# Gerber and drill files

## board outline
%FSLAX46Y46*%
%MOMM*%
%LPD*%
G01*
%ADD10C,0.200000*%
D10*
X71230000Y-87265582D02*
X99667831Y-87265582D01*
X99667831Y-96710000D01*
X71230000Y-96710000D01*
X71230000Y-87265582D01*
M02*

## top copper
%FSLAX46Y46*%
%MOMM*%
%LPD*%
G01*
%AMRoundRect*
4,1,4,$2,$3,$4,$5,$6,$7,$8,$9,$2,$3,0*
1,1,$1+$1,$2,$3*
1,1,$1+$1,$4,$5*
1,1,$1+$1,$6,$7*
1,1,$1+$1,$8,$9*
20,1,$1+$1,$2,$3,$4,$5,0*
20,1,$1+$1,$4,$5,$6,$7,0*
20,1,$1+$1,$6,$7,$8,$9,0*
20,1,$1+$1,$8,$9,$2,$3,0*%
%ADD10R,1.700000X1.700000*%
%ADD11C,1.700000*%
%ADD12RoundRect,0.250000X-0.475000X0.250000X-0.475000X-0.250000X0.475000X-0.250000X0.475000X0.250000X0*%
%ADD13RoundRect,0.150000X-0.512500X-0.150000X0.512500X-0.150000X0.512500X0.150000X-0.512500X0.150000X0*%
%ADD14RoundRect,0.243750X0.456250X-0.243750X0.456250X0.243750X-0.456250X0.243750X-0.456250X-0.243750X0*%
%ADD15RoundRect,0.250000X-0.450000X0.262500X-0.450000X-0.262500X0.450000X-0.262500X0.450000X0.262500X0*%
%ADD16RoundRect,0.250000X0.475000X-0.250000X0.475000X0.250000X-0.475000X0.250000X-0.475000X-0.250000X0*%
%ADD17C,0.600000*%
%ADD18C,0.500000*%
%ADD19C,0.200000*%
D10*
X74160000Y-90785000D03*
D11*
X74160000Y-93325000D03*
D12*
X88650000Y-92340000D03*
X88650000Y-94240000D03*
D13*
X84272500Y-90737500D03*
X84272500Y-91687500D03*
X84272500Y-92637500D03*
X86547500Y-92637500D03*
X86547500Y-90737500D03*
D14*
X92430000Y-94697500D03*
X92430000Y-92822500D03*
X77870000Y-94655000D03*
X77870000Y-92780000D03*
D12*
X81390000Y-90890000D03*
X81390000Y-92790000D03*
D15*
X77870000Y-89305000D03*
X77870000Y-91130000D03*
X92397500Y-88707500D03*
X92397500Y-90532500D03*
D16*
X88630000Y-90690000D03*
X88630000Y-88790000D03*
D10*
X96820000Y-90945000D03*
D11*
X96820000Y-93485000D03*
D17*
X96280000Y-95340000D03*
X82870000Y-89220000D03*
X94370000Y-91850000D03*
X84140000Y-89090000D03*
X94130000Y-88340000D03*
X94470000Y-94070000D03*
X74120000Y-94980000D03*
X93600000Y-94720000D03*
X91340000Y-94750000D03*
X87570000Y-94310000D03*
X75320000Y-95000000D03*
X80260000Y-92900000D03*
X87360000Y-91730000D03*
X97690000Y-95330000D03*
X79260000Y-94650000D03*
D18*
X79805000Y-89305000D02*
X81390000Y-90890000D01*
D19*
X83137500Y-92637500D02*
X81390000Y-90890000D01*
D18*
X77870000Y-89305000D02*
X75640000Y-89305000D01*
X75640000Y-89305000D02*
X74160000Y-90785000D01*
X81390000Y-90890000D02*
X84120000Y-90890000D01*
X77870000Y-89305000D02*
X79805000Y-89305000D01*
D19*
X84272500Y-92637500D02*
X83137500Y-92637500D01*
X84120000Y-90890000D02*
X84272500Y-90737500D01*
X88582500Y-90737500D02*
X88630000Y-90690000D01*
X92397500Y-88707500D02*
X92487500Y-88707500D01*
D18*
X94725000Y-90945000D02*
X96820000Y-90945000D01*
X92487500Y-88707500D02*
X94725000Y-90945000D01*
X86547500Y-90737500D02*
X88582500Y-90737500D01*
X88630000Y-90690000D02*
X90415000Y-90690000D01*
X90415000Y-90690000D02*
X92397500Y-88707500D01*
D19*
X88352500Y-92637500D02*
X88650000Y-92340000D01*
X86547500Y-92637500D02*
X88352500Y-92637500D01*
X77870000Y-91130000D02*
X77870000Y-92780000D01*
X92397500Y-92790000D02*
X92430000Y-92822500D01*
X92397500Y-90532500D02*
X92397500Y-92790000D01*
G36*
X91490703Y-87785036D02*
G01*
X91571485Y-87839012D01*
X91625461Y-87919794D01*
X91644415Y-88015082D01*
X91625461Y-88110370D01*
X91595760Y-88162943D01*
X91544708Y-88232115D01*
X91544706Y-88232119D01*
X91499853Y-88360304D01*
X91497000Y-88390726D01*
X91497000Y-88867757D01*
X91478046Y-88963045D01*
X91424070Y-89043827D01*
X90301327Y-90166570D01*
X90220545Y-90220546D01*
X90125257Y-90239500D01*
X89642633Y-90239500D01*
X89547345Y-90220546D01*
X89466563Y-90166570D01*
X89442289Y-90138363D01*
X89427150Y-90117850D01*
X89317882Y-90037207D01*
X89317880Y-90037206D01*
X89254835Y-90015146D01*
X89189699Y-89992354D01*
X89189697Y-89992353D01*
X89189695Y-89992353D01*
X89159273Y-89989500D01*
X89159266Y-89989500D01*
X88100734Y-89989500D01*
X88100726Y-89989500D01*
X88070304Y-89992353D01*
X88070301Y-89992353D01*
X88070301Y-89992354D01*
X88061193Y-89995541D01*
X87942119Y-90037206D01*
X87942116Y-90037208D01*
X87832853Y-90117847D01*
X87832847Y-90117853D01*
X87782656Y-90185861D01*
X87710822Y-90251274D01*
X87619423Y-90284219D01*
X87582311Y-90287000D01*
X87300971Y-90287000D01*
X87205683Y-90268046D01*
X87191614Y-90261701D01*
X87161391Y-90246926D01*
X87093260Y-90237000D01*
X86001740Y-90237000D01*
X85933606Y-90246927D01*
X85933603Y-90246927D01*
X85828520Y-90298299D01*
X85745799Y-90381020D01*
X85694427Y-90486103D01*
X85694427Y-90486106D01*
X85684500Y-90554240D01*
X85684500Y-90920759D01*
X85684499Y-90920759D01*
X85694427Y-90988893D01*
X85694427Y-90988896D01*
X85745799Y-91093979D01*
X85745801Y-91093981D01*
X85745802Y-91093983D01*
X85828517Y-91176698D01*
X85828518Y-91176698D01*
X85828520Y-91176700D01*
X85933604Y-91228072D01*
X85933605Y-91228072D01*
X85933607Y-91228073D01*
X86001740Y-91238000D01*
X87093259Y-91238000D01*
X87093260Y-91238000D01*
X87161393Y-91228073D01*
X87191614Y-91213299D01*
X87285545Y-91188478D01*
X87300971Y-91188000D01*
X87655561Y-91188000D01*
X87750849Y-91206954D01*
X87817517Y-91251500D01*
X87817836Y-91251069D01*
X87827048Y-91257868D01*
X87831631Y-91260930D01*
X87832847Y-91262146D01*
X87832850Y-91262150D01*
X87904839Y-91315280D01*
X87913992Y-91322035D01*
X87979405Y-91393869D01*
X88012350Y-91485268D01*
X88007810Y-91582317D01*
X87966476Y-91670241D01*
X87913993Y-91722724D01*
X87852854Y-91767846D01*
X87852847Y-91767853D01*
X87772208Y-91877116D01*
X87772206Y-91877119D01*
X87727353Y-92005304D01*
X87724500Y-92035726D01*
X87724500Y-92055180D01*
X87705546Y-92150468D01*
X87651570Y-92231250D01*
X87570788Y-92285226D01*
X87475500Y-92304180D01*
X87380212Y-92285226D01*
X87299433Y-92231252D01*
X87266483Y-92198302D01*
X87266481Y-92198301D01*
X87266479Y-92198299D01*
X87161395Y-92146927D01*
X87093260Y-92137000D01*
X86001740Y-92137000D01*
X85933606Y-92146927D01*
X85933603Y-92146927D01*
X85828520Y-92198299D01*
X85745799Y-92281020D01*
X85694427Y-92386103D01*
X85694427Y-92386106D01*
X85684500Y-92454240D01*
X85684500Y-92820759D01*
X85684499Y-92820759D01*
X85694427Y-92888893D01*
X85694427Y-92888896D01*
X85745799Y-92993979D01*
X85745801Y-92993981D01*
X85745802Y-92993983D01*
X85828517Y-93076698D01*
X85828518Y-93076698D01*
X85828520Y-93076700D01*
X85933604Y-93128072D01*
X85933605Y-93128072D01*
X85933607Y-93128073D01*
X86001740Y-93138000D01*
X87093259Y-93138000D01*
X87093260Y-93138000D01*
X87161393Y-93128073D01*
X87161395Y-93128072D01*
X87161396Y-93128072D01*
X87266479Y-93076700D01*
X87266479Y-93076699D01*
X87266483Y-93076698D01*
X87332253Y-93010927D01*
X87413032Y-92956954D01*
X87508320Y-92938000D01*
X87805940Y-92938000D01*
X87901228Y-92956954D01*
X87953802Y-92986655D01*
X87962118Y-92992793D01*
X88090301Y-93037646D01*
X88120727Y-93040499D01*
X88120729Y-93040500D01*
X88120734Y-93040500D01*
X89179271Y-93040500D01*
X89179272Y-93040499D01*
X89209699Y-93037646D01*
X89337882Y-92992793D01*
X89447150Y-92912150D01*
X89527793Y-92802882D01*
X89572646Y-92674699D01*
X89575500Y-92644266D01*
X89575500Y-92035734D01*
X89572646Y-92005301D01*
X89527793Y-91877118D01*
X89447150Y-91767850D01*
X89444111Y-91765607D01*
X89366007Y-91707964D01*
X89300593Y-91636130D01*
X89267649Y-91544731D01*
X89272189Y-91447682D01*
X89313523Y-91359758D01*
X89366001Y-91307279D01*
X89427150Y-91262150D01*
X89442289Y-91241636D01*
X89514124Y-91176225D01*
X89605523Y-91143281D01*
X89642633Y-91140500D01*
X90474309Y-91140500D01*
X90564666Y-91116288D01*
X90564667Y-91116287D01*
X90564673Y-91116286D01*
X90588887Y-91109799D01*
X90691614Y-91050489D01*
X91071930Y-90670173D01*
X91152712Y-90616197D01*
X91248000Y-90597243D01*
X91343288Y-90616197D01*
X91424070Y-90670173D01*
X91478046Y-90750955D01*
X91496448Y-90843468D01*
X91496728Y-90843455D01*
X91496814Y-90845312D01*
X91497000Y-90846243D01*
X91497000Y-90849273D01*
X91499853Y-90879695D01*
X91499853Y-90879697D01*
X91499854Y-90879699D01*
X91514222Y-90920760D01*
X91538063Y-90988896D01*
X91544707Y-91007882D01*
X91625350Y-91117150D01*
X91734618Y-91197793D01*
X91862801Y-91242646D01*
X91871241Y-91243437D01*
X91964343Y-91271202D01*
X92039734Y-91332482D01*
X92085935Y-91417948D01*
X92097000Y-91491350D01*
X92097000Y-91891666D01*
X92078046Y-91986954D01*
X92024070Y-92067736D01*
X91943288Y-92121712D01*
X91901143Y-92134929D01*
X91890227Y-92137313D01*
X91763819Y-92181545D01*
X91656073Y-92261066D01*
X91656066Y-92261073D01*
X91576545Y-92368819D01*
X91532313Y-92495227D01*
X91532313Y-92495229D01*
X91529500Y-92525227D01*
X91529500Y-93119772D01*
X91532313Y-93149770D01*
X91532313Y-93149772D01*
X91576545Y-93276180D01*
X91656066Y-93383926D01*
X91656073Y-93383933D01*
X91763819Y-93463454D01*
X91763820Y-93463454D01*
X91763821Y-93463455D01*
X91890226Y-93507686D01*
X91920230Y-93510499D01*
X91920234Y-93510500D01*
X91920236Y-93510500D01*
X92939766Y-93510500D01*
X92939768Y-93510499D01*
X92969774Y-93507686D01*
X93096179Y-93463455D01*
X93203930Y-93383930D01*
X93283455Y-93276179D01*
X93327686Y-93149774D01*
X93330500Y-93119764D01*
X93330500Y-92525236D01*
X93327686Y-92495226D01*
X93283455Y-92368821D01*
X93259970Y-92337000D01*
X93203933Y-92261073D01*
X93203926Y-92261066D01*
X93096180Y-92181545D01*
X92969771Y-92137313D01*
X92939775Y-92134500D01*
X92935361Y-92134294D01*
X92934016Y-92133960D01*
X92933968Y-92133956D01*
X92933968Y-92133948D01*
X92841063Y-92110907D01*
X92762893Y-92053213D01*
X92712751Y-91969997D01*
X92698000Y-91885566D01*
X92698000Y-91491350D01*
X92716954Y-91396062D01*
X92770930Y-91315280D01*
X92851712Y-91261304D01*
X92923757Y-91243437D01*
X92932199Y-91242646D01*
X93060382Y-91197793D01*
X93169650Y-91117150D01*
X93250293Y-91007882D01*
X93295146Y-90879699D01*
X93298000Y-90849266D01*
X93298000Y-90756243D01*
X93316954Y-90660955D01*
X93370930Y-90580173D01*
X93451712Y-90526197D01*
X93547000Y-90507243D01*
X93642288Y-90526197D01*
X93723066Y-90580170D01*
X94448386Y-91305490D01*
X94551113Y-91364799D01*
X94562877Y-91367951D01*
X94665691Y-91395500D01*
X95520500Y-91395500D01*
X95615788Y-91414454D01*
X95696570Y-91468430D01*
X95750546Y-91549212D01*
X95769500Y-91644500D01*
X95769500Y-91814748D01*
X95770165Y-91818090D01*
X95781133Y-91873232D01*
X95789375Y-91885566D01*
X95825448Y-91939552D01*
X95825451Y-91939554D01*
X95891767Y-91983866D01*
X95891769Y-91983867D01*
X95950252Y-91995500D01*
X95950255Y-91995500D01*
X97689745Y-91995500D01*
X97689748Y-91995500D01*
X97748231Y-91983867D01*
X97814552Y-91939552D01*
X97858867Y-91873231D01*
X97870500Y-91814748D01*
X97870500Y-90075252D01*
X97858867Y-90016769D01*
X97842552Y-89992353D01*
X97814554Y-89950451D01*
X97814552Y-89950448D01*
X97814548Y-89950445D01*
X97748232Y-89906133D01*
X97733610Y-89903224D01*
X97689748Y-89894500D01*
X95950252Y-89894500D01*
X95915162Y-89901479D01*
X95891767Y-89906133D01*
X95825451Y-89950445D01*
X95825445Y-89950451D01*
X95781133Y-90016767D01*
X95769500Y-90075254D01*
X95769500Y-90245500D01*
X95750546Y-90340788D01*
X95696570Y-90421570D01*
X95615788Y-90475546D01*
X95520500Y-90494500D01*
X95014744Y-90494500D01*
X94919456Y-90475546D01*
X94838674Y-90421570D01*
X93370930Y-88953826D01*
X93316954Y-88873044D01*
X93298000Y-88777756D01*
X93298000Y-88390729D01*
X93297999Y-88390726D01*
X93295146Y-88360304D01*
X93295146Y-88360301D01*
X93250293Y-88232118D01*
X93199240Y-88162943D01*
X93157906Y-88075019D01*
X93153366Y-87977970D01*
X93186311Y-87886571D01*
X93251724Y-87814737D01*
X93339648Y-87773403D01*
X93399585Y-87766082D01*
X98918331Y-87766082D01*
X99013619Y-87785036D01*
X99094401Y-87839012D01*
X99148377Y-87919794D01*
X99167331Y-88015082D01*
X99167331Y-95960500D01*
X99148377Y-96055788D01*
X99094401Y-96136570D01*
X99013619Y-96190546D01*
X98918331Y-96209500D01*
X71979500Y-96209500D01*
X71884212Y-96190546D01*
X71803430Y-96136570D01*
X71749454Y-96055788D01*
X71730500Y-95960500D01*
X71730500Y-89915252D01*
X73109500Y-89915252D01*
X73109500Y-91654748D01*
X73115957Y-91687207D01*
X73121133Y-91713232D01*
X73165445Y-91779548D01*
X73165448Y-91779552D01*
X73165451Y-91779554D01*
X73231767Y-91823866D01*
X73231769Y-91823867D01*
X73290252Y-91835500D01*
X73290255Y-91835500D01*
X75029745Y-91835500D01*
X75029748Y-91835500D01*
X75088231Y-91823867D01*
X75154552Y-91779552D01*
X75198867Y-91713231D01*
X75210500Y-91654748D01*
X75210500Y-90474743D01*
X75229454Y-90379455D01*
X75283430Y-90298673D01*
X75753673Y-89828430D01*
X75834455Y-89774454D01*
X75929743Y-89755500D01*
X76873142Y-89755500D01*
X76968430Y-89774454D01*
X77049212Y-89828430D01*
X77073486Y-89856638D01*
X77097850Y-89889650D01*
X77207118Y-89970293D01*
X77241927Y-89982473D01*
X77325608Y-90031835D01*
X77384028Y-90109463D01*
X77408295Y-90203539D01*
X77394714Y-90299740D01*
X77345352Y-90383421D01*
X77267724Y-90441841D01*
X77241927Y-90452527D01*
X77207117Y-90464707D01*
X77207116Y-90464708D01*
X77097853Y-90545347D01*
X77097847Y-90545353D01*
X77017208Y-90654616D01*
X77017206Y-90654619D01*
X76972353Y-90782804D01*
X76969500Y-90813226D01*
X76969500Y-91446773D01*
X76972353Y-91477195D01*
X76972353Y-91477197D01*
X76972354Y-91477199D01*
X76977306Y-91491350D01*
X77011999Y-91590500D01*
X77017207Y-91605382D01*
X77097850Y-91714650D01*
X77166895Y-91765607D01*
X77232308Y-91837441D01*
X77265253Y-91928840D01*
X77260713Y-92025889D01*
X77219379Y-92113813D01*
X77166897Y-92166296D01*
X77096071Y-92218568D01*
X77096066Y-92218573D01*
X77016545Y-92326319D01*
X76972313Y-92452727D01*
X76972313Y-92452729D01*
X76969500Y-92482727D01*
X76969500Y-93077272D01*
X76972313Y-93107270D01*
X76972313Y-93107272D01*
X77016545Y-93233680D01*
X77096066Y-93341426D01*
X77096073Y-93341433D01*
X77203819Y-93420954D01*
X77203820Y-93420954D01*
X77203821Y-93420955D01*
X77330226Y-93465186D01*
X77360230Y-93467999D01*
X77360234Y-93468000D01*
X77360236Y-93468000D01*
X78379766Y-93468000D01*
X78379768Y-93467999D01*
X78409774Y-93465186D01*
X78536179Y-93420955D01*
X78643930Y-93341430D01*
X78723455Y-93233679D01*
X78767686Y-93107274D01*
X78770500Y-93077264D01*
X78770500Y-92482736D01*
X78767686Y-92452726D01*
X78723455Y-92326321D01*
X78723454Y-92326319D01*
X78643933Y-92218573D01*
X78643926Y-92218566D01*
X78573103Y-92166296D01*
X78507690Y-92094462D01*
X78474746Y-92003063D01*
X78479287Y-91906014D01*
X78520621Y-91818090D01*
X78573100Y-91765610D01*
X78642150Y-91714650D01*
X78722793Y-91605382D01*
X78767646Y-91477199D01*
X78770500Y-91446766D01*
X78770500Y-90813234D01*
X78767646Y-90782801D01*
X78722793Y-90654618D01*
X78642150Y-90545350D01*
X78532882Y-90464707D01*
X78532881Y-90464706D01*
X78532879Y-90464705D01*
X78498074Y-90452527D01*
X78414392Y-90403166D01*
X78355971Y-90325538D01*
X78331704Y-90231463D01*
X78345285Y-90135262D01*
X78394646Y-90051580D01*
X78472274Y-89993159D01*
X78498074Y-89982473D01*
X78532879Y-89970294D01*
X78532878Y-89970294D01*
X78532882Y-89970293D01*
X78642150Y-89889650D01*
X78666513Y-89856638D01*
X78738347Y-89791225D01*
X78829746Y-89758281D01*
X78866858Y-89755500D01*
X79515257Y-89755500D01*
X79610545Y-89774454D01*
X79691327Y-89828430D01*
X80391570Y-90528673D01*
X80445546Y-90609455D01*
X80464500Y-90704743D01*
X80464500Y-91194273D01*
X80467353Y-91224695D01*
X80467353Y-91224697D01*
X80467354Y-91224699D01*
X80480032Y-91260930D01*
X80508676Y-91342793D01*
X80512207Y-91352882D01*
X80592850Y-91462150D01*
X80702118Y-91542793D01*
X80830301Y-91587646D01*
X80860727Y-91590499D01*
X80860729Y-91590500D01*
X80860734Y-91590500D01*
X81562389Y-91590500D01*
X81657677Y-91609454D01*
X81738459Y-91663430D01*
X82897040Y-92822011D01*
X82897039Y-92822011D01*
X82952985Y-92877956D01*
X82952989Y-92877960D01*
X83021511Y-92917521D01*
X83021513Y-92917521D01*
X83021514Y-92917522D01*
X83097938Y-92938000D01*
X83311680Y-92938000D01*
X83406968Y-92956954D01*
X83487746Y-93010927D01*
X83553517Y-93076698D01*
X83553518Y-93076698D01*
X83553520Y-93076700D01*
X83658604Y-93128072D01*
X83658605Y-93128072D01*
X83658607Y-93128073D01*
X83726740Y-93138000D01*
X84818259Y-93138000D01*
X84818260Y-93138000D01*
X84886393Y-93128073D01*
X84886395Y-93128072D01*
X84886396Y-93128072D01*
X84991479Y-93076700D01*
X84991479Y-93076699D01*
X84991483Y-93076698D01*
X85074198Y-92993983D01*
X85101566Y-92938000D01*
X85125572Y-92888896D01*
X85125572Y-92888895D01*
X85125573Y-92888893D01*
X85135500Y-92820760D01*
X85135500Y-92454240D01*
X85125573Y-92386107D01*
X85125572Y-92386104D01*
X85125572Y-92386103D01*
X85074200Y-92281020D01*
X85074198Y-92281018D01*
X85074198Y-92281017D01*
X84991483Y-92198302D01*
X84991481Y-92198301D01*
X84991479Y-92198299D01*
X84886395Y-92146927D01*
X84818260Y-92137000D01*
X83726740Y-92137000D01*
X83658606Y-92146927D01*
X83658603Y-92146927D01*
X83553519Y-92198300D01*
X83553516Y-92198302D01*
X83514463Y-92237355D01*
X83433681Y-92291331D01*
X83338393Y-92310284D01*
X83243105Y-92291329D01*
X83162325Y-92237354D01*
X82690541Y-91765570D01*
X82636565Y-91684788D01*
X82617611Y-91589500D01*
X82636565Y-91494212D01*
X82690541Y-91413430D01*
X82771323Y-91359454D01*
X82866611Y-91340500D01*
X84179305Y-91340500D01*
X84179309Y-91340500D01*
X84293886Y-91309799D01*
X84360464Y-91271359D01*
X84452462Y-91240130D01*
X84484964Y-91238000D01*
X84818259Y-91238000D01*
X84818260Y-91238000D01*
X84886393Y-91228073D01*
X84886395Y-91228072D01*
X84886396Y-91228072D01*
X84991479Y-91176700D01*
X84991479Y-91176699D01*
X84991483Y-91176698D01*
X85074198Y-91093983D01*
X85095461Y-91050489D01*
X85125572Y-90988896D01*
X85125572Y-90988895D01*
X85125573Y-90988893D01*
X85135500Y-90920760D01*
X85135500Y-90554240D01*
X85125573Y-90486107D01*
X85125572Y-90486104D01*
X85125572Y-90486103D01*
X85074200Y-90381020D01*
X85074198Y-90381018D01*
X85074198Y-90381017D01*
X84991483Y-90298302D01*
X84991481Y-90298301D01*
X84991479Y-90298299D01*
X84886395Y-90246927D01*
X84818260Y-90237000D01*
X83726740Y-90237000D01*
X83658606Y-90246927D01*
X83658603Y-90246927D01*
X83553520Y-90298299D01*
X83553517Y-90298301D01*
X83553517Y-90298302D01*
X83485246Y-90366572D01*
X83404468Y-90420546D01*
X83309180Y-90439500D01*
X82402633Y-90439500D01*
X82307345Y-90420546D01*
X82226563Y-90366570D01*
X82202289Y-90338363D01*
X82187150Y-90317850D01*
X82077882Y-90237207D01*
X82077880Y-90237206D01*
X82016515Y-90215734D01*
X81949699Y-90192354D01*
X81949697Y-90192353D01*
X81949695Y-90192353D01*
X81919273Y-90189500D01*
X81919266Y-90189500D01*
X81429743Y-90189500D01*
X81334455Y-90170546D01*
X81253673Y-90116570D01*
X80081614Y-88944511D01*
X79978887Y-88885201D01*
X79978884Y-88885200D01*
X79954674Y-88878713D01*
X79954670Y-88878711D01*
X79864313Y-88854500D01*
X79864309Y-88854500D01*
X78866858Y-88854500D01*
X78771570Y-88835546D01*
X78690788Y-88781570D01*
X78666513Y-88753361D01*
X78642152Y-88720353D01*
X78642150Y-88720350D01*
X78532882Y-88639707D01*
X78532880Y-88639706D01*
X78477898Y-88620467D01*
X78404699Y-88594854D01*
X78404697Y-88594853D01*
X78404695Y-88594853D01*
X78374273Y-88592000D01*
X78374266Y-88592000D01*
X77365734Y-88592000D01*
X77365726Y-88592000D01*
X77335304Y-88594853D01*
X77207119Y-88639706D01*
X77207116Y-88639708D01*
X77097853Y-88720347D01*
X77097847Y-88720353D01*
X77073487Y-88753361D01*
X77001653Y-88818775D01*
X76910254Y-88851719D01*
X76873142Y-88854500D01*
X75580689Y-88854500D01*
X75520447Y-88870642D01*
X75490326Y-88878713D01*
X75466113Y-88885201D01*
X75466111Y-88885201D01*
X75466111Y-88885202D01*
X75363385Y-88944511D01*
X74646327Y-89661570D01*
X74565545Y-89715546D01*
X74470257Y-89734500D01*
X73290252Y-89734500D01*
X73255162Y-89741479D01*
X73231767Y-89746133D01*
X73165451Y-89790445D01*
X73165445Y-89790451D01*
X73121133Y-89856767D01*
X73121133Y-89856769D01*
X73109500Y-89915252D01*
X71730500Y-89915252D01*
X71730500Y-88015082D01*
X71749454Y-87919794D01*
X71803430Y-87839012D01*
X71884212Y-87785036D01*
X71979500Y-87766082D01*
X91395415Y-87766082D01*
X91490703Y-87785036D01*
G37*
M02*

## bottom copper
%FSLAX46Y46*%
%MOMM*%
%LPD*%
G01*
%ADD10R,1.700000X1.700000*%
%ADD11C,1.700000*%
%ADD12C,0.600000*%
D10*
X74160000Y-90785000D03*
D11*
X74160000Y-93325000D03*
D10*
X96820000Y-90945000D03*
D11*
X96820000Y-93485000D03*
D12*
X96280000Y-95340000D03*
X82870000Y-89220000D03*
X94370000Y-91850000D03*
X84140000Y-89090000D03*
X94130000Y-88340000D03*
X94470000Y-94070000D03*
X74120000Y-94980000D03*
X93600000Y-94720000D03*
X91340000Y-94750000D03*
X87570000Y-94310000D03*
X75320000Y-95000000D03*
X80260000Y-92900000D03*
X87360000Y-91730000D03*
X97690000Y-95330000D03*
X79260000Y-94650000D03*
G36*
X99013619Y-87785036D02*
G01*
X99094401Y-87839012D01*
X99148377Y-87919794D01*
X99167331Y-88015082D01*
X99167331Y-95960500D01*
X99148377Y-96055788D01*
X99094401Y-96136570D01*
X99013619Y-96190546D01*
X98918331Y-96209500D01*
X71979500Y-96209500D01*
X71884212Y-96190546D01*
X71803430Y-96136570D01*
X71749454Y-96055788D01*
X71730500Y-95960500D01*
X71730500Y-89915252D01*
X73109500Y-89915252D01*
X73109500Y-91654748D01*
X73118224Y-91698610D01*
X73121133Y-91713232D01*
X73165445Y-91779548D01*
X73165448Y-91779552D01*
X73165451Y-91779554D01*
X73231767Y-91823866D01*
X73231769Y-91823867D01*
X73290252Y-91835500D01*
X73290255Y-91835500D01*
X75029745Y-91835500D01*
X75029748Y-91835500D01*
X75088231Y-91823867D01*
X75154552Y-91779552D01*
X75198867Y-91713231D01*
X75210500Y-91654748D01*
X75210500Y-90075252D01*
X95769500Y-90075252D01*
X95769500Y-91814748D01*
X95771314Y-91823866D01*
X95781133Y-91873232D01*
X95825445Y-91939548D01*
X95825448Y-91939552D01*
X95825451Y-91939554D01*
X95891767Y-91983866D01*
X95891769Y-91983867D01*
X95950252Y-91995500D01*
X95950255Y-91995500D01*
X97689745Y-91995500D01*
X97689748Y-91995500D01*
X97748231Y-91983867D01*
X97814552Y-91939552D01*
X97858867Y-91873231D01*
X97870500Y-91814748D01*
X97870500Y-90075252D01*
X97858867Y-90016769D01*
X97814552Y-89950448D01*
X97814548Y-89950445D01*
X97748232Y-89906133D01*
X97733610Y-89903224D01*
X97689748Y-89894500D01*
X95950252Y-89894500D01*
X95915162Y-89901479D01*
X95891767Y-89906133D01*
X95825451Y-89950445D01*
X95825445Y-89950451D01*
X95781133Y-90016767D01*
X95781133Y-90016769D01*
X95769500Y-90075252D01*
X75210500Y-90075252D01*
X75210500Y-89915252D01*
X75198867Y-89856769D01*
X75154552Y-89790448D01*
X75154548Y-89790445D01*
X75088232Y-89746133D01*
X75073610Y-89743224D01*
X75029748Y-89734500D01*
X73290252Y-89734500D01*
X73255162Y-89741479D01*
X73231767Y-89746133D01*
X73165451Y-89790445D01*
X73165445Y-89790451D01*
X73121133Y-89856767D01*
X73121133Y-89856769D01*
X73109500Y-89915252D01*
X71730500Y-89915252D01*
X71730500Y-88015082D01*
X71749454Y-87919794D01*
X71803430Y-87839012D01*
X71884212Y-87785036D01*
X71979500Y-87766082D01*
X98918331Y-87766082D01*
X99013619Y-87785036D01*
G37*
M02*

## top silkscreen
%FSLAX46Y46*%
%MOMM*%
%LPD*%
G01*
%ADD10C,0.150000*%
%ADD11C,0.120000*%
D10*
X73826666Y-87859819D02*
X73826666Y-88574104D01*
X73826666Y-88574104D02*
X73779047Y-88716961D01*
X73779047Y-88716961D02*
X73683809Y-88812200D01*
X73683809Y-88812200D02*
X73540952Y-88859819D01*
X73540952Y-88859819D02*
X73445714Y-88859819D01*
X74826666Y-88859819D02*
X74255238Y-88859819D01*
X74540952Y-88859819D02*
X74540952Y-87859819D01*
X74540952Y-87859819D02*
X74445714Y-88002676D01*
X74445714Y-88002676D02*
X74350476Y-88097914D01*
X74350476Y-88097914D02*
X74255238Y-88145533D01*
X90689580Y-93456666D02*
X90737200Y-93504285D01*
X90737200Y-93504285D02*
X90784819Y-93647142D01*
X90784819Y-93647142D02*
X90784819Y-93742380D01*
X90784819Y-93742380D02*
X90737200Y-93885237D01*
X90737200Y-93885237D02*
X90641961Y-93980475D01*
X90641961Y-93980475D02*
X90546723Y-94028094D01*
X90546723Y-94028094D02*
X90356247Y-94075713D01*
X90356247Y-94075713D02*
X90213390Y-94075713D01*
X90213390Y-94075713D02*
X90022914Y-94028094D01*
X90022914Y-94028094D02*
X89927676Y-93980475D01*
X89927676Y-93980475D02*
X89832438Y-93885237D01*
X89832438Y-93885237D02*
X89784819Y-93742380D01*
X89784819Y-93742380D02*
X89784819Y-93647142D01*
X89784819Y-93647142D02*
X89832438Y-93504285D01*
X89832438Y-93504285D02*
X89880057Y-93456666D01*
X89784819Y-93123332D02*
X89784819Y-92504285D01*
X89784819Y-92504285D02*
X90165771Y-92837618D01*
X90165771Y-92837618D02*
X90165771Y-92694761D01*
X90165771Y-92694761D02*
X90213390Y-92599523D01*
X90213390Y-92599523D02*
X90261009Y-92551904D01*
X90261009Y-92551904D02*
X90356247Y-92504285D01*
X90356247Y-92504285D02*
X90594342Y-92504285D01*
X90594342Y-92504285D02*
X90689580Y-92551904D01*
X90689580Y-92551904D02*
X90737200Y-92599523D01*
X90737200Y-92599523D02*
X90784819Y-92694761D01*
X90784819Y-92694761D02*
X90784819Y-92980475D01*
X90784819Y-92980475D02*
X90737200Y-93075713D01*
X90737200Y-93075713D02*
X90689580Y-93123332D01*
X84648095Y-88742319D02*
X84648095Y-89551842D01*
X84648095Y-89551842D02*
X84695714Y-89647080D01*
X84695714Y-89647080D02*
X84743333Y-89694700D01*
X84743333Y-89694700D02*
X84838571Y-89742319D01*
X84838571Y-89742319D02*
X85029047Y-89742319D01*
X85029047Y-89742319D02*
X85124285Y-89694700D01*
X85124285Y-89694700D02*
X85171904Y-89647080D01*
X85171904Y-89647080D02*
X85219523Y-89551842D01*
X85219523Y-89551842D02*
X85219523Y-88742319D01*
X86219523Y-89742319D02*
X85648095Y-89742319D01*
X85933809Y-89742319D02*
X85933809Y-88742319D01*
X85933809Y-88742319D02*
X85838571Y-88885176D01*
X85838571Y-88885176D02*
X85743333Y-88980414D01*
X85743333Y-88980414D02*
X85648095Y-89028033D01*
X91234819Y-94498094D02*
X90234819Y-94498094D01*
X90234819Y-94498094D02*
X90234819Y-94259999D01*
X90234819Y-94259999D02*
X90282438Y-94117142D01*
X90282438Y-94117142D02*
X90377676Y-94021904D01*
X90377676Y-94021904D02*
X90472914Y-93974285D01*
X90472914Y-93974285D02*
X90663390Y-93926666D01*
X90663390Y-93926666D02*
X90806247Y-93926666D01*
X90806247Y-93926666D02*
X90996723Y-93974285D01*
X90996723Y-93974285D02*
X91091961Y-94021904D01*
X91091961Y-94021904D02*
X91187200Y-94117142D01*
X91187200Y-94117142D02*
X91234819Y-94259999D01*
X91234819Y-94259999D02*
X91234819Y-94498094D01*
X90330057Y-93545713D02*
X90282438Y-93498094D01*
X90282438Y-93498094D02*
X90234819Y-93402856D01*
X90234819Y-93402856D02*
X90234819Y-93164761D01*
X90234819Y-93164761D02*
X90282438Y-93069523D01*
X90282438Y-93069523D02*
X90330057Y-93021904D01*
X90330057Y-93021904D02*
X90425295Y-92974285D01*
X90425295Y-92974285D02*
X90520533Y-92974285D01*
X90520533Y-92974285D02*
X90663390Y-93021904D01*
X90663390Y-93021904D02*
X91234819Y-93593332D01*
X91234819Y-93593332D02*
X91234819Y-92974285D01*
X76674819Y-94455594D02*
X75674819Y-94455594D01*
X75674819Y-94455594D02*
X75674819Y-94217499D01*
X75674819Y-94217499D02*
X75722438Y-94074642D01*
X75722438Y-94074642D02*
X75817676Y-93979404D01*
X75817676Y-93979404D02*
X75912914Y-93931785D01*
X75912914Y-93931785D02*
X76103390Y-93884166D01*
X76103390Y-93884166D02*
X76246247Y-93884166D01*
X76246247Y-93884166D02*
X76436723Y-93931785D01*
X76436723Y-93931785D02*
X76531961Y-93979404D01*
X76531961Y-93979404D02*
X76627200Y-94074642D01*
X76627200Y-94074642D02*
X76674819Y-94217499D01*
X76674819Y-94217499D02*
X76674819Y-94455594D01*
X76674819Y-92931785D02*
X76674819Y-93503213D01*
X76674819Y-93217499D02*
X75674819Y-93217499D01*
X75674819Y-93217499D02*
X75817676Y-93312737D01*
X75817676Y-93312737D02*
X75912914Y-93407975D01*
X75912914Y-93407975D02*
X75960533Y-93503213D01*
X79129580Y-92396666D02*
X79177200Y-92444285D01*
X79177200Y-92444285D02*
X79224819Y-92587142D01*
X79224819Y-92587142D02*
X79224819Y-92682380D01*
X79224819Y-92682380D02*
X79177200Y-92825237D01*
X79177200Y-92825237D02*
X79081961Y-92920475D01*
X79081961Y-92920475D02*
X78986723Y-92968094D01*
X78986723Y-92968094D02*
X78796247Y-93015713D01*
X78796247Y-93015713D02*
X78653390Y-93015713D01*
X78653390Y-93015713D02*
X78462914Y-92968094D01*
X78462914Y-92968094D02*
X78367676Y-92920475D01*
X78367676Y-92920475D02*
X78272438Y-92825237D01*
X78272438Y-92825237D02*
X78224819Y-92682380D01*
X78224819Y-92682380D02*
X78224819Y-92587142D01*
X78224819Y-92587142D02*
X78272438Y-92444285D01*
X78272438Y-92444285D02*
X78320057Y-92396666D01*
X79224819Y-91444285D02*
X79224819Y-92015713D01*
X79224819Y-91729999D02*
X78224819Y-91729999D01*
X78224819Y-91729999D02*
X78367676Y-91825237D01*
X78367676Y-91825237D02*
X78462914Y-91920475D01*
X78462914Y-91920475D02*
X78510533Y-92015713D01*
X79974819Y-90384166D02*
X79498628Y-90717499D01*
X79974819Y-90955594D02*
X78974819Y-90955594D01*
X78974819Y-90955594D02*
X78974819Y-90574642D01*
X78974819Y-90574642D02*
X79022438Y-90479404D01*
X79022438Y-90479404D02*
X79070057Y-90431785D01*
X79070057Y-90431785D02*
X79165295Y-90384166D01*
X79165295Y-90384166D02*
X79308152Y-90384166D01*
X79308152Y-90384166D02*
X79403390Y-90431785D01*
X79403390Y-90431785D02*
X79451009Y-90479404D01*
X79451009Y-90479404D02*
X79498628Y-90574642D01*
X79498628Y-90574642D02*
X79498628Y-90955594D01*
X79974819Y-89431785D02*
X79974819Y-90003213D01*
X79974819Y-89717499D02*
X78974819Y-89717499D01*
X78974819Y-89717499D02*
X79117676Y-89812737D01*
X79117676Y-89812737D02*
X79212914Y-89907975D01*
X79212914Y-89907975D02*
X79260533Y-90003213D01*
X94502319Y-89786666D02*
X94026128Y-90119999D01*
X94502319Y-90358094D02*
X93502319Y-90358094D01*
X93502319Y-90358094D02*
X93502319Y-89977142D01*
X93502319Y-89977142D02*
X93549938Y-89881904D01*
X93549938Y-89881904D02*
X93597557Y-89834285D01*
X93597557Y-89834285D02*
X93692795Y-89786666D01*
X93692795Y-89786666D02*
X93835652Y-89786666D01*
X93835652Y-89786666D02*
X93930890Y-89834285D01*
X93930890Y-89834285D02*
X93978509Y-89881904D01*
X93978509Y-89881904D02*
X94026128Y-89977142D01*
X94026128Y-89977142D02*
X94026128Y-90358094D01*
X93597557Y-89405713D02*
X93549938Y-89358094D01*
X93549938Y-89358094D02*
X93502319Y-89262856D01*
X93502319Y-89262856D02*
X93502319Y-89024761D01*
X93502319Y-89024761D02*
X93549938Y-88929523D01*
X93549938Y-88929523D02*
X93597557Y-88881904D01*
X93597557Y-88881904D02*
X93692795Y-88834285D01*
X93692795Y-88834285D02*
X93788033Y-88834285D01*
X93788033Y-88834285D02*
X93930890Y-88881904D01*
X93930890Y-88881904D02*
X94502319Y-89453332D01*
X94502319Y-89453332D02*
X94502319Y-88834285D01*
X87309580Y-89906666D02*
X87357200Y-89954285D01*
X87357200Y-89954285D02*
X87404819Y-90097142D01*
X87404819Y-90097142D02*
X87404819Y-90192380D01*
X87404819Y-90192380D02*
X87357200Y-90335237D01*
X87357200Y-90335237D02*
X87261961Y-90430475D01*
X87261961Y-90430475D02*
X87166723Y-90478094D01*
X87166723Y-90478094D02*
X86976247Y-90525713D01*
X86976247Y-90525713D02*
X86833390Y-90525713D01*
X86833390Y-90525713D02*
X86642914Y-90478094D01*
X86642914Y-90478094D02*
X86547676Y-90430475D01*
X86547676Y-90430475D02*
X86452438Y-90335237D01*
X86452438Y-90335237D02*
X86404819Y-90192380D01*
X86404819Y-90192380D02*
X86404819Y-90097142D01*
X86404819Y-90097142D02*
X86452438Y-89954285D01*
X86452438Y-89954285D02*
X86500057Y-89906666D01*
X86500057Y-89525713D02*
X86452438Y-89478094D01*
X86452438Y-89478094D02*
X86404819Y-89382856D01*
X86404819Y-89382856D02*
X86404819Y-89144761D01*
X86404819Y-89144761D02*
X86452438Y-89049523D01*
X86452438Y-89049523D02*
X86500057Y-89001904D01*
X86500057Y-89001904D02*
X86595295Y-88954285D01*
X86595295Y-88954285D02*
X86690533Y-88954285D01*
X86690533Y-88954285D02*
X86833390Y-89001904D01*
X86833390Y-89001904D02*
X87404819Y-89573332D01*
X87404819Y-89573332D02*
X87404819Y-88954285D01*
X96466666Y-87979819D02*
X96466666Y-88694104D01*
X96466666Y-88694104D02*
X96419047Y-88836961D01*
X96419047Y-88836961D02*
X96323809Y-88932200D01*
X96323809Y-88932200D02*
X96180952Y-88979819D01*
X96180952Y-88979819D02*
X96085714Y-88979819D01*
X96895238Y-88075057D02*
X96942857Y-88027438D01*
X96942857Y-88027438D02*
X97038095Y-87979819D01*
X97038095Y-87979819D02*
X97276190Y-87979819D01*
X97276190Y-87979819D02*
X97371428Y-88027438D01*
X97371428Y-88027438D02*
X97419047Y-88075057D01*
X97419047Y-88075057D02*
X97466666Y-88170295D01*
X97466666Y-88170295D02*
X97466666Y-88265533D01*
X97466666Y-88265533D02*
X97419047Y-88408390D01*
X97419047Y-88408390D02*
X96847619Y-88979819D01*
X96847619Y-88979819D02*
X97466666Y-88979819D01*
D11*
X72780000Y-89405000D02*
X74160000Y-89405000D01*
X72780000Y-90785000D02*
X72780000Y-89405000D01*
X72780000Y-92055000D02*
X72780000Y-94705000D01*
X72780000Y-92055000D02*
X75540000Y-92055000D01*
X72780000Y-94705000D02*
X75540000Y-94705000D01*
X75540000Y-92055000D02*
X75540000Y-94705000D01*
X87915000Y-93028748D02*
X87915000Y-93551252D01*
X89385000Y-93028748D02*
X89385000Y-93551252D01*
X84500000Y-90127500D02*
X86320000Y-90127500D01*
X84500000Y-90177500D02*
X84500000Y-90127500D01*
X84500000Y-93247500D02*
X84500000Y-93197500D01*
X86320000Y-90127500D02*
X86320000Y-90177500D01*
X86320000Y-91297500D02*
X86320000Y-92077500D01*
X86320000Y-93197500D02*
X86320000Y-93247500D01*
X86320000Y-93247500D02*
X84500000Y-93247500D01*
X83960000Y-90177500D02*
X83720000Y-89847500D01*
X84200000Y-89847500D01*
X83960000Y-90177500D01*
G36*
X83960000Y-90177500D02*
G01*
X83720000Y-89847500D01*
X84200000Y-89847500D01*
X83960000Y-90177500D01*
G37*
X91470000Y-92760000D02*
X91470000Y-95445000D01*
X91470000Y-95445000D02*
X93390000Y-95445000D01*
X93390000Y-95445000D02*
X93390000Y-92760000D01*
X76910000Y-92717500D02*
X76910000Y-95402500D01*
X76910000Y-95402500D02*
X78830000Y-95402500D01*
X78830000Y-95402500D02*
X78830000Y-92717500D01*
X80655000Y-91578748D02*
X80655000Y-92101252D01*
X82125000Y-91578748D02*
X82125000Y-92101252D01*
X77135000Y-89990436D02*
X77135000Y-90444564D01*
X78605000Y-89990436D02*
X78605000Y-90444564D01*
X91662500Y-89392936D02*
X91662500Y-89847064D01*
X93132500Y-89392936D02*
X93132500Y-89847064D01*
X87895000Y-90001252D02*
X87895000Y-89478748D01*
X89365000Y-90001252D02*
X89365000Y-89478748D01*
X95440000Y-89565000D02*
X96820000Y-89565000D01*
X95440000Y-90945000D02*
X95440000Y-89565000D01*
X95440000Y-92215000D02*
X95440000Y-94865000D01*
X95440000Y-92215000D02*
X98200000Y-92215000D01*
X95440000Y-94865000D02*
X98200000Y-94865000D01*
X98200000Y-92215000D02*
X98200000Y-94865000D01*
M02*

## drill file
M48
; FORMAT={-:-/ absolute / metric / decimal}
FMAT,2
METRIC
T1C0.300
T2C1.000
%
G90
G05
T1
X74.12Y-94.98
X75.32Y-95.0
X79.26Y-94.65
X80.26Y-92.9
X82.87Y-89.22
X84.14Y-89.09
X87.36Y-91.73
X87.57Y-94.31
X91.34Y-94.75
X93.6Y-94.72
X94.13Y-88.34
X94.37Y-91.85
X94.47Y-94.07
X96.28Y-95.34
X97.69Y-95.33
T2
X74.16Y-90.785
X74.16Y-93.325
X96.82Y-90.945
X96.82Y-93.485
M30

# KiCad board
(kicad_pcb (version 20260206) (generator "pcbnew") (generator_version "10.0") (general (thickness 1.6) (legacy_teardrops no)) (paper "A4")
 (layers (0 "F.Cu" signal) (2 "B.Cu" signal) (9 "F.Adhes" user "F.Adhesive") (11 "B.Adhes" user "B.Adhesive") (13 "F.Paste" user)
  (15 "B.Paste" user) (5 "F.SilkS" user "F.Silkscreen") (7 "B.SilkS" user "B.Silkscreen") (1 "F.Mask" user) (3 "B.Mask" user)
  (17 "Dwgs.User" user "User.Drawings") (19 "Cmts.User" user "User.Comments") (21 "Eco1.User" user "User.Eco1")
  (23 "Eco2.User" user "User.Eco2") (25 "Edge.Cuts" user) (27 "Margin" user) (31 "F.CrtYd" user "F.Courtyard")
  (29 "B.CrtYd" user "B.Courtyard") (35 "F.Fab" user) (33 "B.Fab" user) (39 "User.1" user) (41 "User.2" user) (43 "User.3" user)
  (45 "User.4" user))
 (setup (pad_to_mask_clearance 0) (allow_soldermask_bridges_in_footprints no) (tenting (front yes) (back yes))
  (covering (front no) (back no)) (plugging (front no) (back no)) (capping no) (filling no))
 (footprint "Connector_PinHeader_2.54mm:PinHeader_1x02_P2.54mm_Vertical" (layer "F.Cu") (at 74.16 90.785)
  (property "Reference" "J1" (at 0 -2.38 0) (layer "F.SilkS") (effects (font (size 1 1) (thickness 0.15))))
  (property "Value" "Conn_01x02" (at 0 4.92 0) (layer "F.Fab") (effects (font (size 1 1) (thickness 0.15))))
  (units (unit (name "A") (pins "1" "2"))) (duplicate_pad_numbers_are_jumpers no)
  (fp_line (start -1.38 -1.38) (end 0 -1.38) (stroke (width 0.12) (type solid)) (layer "F.SilkS"))
  (fp_line (start -1.38 0) (end -1.38 -1.38) (stroke (width 0.12) (type solid)) (layer "F.SilkS"))
  (fp_line (start -1.38 1.27) (end -1.38 3.92) (stroke (width 0.12) (type solid)) (layer "F.SilkS"))
  (fp_line (start -1.38 1.27) (end 1.38 1.27) (stroke (width 0.12) (type solid)) (layer "F.SilkS"))
  (fp_line (start -1.38 3.92) (end 1.38 3.92) (stroke (width 0.12) (type solid)) (layer "F.SilkS"))
  (fp_line (start 1.38 1.27) (end 1.38 3.92) (stroke (width 0.12) (type solid)) (layer "F.SilkS"))
  (pad "1" thru_hole rect (at 0 0) (size 1.7 1.7) (drill 1) (layers "*.Cu" "*.Mask") (remove_unused_layers no) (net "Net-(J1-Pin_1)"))
  (pad "2" thru_hole circle (at 0 2.54) (size 1.7 1.7) (drill 1) (layers "*.Cu" "*.Mask") (remove_unused_layers no) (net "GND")))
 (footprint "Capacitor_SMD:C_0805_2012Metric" (layer "F.Cu") (at 88.65 93.29 -90)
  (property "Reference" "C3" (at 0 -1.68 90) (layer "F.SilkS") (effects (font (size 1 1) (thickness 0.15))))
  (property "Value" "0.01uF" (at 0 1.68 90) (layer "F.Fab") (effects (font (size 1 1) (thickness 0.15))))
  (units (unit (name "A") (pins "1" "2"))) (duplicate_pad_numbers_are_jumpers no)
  (fp_line (start -0.261252 0.735) (end 0.261252 0.735) (stroke (width 0.12) (type solid)) (layer "F.SilkS"))
  (fp_line (start -0.261252 -0.735) (end 0.261252 -0.735) (stroke (width 0.12) (type solid)) (layer "F.SilkS"))
  (pad "1" smd roundrect (at -0.95 0 270) (size 1 1.45) (layers "F.Cu" "F.Mask" "F.Paste") (roundrect_rratio 0.25) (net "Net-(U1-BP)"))
  (pad "2" smd roundrect (at 0.95 0 270) (size 1 1.45) (layers "F.Cu" "F.Mask" "F.Paste") (roundrect_rratio 0.25) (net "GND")))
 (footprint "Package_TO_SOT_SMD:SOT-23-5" (layer "F.Cu") (at 85.41 91.6875)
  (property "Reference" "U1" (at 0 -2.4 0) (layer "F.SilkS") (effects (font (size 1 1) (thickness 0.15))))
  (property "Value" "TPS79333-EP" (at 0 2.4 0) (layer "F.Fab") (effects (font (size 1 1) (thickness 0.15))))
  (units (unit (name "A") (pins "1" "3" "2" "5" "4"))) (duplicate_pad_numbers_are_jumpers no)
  (fp_line (start -0.91 -1.56) (end 0.91 -1.56) (stroke (width 0.12) (type solid)) (layer "F.SilkS"))
  (fp_line (start -0.91 -1.51) (end -0.91 -1.56) (stroke (width 0.12) (type solid)) (layer "F.SilkS"))
  (fp_line (start -0.91 1.56) (end -0.91 1.51) (stroke (width 0.12) (type solid)) (layer "F.SilkS"))
  (fp_line (start 0.91 -1.56) (end 0.91 -1.51) (stroke (width 0.12) (type solid)) (layer "F.SilkS"))
  (fp_line (start 0.91 -0.39) (end 0.91 0.39) (stroke (width 0.12) (type solid)) (layer "F.SilkS"))
  (fp_line (start 0.91 1.51) (end 0.91 1.56) (stroke (width 0.12) (type solid)) (layer "F.SilkS"))
  (fp_line (start 0.91 1.56) (end -0.91 1.56) (stroke (width 0.12) (type solid)) (layer "F.SilkS"))
  (fp_poly (pts (xy -1.45 -1.51) (xy -1.69 -1.84) (xy -1.21 -1.84)) (stroke (width 0.12) (type solid)) (fill yes) (layer "F.SilkS"))
  (pad "1" smd roundrect (at -1.1375 -0.95) (size 1.325 0.6) (layers "F.Cu" "F.Mask" "F.Paste") (roundrect_rratio 0.25)
   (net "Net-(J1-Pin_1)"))
  (pad "2" smd roundrect (at -1.1375 0) (size 1.325 0.6) (layers "F.Cu" "F.Mask" "F.Paste") (roundrect_rratio 0.25) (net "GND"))
  (pad "3" smd roundrect (at -1.1375 0.95) (size 1.325 0.6) (layers "F.Cu" "F.Mask" "F.Paste") (roundrect_rratio 0.25)
   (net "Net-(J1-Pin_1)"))
  (pad "4" smd roundrect (at 1.1375 0.95) (size 1.325 0.6) (layers "F.Cu" "F.Mask" "F.Paste") (roundrect_rratio 0.25) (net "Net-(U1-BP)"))
  (pad "5" smd roundrect (at 1.1375 -0.95) (size 1.325 0.6) (layers "F.Cu" "F.Mask" "F.Paste") (roundrect_rratio 0.25)
   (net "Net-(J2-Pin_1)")))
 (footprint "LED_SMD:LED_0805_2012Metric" (layer "F.Cu") (at 92.43 93.76 90)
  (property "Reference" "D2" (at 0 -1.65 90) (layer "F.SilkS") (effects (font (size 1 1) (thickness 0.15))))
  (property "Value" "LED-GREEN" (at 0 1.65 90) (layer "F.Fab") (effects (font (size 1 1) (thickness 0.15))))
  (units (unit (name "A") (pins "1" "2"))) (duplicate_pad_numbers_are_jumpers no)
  (fp_line (start 1 -0.96) (end -1.685 -0.96) (stroke (width 0.12) (type solid)) (layer "F.SilkS"))
  (fp_line (start -1.685 -0.96) (end -1.685 0.96) (stroke (width 0.12) (type solid)) (layer "F.SilkS"))
  (fp_line (start -1.685 0.96) (end 1 0.96) (stroke (width 0.12) (type solid)) (layer "F.SilkS"))
  (pad "1" smd roundrect (at -0.9375 0 90) (size 0.975 1.4) (layers "F.Cu" "F.Mask" "F.Paste") (roundrect_rratio 0.25) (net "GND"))
  (pad "2" smd roundrect (at 0.9375 0 90) (size 0.975 1.4) (layers "F.Cu" "F.Mask" "F.Paste") (roundrect_rratio 0.25) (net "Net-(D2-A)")))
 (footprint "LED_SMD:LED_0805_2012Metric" (layer "F.Cu") (at 77.87 93.7175 90)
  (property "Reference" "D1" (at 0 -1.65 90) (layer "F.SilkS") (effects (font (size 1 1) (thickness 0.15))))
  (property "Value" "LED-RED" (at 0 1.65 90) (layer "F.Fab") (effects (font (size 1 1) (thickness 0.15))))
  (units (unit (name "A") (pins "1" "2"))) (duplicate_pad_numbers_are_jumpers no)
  (fp_line (start 1 -0.96) (end -1.685 -0.96) (stroke (width 0.12) (type solid)) (layer "F.SilkS"))
  (fp_line (start -1.685 -0.96) (end -1.685 0.96) (stroke (width 0.12) (type solid)) (layer "F.SilkS"))
  (fp_line (start -1.685 0.96) (end 1 0.96) (stroke (width 0.12) (type solid)) (layer "F.SilkS"))
  (pad "1" smd roundrect (at -0.9375 0 90) (size 0.975 1.4) (layers "F.Cu" "F.Mask" "F.Paste") (roundrect_rratio 0.25) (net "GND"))
  (pad "2" smd roundrect (at 0.9375 0 90) (size 0.975 1.4) (layers "F.Cu" "F.Mask" "F.Paste") (roundrect_rratio 0.25) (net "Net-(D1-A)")))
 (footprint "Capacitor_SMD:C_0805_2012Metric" (layer "F.Cu") (at 81.39 91.84 -90)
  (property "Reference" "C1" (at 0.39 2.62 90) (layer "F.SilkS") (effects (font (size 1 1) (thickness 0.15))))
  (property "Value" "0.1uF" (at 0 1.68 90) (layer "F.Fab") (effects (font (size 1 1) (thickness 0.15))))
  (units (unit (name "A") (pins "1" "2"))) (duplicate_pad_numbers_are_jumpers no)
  (fp_line (start -0.261252 0.735) (end 0.261252 0.735) (stroke (width 0.12) (type solid)) (layer "F.SilkS"))
  (fp_line (start -0.261252 -0.735) (end 0.261252 -0.735) (stroke (width 0.12) (type solid)) (layer "F.SilkS"))
  (pad "1" smd roundrect (at -0.95 0 270) (size 1 1.45) (layers "F.Cu" "F.Mask" "F.Paste") (roundrect_rratio 0.25) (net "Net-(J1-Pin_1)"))
  (pad "2" smd roundrect (at 0.95 0 270) (size 1 1.45) (layers "F.Cu" "F.Mask" "F.Paste") (roundrect_rratio 0.25) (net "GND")))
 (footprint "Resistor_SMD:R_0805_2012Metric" (layer "F.Cu") (at 77.87 90.2175 -90)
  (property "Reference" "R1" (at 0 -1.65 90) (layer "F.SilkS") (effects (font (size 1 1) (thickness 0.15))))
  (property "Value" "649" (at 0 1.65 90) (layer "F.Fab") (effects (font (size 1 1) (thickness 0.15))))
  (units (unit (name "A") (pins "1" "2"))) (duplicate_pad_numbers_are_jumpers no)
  (fp_line (start -0.227064 0.735) (end 0.227064 0.735) (stroke (width 0.12) (type solid)) (layer "F.SilkS"))
  (fp_line (start -0.227064 -0.735) (end 0.227064 -0.735) (stroke (width 0.12) (type solid)) (layer "F.SilkS"))
  (pad "1" smd roundrect (at -0.9125 0 270) (size 1.025 1.4) (layers "F.Cu" "F.Mask" "F.Paste") (roundrect_rratio 0.243902)
   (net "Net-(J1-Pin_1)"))
  (pad "2" smd roundrect (at 0.9125 0 270) (size 1.025 1.4) (layers "F.Cu" "F.Mask" "F.Paste") (roundrect_rratio 0.243902)
   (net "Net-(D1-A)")))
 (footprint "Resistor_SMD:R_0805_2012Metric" (layer "F.Cu") (at 92.3975 89.62 -90)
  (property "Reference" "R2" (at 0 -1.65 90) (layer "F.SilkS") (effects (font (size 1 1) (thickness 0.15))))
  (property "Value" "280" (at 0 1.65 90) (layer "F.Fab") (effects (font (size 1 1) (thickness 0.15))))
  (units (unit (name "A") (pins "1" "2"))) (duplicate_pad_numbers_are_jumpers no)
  (fp_line (start -0.227064 0.735) (end 0.227064 0.735) (stroke (width 0.12) (type solid)) (layer "F.SilkS"))
  (fp_line (start -0.227064 -0.735) (end 0.227064 -0.735) (stroke (width 0.12) (type solid)) (layer "F.SilkS"))
  (pad "1" smd roundrect (at -0.9125 0 270) (size 1.025 1.4) (layers "F.Cu" "F.Mask" "F.Paste") (roundrect_rratio 0.243902)
   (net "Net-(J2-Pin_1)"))
  (pad "2" smd roundrect (at 0.9125 0 270) (size 1.025 1.4) (layers "F.Cu" "F.Mask" "F.Paste") (roundrect_rratio 0.243902)
   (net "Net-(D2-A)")))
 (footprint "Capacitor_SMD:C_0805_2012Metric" (layer "F.Cu") (at 88.63 89.74 90)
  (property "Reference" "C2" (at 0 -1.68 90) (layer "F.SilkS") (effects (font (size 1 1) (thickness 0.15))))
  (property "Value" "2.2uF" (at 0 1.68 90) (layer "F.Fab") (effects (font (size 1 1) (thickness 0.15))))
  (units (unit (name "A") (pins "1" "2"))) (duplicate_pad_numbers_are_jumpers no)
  (fp_line (start -0.261252 -0.735) (end 0.261252 -0.735) (stroke (width 0.12) (type solid)) (layer "F.SilkS"))
  (fp_line (start -0.261252 0.735) (end 0.261252 0.735) (stroke (width 0.12) (type solid)) (layer "F.SilkS"))
  (pad "1" smd roundrect (at -0.95 0 90) (size 1 1.45) (layers "F.Cu" "F.Mask" "F.Paste") (roundrect_rratio 0.25) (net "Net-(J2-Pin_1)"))
  (pad "2" smd roundrect (at 0.95 0 90) (size 1 1.45) (layers "F.Cu" "F.Mask" "F.Paste") (roundrect_rratio 0.25) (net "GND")))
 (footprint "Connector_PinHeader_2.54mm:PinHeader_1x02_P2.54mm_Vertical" (layer "F.Cu") (at 96.82 90.945)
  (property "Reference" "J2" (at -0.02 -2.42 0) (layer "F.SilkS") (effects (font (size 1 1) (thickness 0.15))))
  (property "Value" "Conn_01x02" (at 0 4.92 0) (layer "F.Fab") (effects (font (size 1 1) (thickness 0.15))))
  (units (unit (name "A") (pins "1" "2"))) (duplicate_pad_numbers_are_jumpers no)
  (fp_line (start -1.38 -1.38) (end 0 -1.38) (stroke (width 0.12) (type solid)) (layer "F.SilkS"))
  (fp_line (start -1.38 0) (end -1.38 -1.38) (stroke (width 0.12) (type solid)) (layer "F.SilkS"))
  (fp_line (start -1.38 1.27) (end -1.38 3.92) (stroke (width 0.12) (type solid)) (layer "F.SilkS"))
  (fp_line (start -1.38 1.27) (end 1.38 1.27) (stroke (width 0.12) (type solid)) (layer "F.SilkS"))
  (fp_line (start -1.38 3.92) (end 1.38 3.92) (stroke (width 0.12) (type solid)) (layer "F.SilkS"))
  (fp_line (start 1.38 1.27) (end 1.38 3.92) (stroke (width 0.12) (type solid)) (layer "F.SilkS"))
  (pad "1" thru_hole rect (at 0 0) (size 1.7 1.7) (drill 1) (layers "*.Cu" "*.Mask") (remove_unused_layers no) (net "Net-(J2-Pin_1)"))
  (pad "2" thru_hole circle (at 0 2.54) (size 1.7 1.7) (drill 1) (layers "*.Cu" "*.Mask") (remove_unused_layers no) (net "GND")))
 (gr_rect (start 71.23 87.265582) (end 99.667831 96.71) (stroke (width 0.2) (type solid)) (fill no) (layer "Edge.Cuts"))
 (via (at 96.28 95.34) (size 0.6) (drill 0.3) (layers "F.Cu" "B.Cu") (free yes) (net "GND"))
 (via (at 82.87 89.22) (size 0.6) (drill 0.3) (layers "F.Cu" "B.Cu") (free yes) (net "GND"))
 (via (at 94.37 91.85) (size 0.6) (drill 0.3) (layers "F.Cu" "B.Cu") (free yes) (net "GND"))
 (via (at 84.14 89.09) (size 0.6) (drill 0.3) (layers "F.Cu" "B.Cu") (free yes) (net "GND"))
 (via (at 94.13 88.34) (size 0.6) (drill 0.3) (layers "F.Cu" "B.Cu") (free yes) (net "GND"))
 (via (at 94.47 94.07) (size 0.6) (drill 0.3) (layers "F.Cu" "B.Cu") (free yes) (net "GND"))
 (via (at 74.12 94.98) (size 0.6) (drill 0.3) (layers "F.Cu" "B.Cu") (free yes) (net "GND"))
 (via (at 93.6 94.72) (size 0.6) (drill 0.3) (layers "F.Cu" "B.Cu") (free yes) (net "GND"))
 (via (at 91.34 94.75) (size 0.6) (drill 0.3) (layers "F.Cu" "B.Cu") (free yes) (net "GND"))
 (via (at 87.57 94.31) (size 0.6) (drill 0.3) (layers "F.Cu" "B.Cu") (free yes) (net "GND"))
 (via (at 75.32 95) (size 0.6) (drill 0.3) (layers "F.Cu" "B.Cu") (free yes) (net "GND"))
 (via (at 80.26 92.9) (size 0.6) (drill 0.3) (layers "F.Cu" "B.Cu") (free yes) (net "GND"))
 (via (at 87.36 91.73) (size 0.6) (drill 0.3) (layers "F.Cu" "B.Cu") (free yes) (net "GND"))
 (via (at 97.69 95.33) (size 0.6) (drill 0.3) (layers "F.Cu" "B.Cu") (free yes) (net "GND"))
 (via (at 79.26 94.65) (size 0.6) (drill 0.3) (layers "F.Cu" "B.Cu") (free yes) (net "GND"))
 (segment (start 79.805 89.305) (end 81.39 90.89) (width 0.5) (layer "F.Cu") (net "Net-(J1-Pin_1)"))
 (segment (start 83.1375 92.6375) (end 81.39 90.89) (width 0.2) (layer "F.Cu") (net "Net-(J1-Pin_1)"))
 (segment (start 77.87 89.305) (end 75.64 89.305) (width 0.5) (layer "F.Cu") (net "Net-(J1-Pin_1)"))
 (segment (start 75.64 89.305) (end 74.16 90.785) (width 0.5) (layer "F.Cu") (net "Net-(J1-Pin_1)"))
 (segment (start 81.39 90.89) (end 84.12 90.89) (width 0.5) (layer "F.Cu") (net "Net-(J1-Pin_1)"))
 (segment (start 77.87 89.305) (end 79.805 89.305) (width 0.5) (layer "F.Cu") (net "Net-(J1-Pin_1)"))
 (segment (start 84.2725 92.6375) (end 83.1375 92.6375) (width 0.2) (layer "F.Cu") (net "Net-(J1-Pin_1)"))
 (segment (start 84.12 90.89) (end 84.2725 90.7375) (width 0.2) (layer "F.Cu") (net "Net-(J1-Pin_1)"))
 (segment (start 88.5825 90.7375) (end 88.63 90.69) (width 0.2) (layer "F.Cu") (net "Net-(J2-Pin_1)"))
 (segment (start 92.3975 88.7075) (end 92.4875 88.7075) (width 0.2) (layer "F.Cu") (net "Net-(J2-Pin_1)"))
 (segment (start 94.725 90.945) (end 96.82 90.945) (width 0.5) (layer "F.Cu") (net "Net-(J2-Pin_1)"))
 (segment (start 92.4875 88.7075) (end 94.725 90.945) (width 0.5) (layer "F.Cu") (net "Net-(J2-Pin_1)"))
 (segment (start 86.5475 90.7375) (end 88.5825 90.7375) (width 0.5) (layer "F.Cu") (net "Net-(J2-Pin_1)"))
 (segment (start 88.63 90.69) (end 90.415 90.69) (width 0.5) (layer "F.Cu") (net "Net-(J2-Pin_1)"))
 (segment (start 90.415 90.69) (end 92.3975 88.7075) (width 0.5) (layer "F.Cu") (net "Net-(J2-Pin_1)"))
 (segment (start 88.3525 92.6375) (end 88.65 92.34) (width 0.2) (layer "F.Cu") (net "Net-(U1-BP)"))
 (segment (start 86.5475 92.6375) (end 88.3525 92.6375) (width 0.2) (layer "F.Cu") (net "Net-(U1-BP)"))
 (segment (start 77.87 91.13) (end 77.87 92.78) (width 0.2) (layer "F.Cu") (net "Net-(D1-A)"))
 (segment (start 92.3975 92.79) (end 92.43 92.8225) (width 0.2) (layer "F.Cu") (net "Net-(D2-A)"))
 (segment (start 92.3975 90.5325) (end 92.3975 92.79) (width 0.2) (layer "F.Cu") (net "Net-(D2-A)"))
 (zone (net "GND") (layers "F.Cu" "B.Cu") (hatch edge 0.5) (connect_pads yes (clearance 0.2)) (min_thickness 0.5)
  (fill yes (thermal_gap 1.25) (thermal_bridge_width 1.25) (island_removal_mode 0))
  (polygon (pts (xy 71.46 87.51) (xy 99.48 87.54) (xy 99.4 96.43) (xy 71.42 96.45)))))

